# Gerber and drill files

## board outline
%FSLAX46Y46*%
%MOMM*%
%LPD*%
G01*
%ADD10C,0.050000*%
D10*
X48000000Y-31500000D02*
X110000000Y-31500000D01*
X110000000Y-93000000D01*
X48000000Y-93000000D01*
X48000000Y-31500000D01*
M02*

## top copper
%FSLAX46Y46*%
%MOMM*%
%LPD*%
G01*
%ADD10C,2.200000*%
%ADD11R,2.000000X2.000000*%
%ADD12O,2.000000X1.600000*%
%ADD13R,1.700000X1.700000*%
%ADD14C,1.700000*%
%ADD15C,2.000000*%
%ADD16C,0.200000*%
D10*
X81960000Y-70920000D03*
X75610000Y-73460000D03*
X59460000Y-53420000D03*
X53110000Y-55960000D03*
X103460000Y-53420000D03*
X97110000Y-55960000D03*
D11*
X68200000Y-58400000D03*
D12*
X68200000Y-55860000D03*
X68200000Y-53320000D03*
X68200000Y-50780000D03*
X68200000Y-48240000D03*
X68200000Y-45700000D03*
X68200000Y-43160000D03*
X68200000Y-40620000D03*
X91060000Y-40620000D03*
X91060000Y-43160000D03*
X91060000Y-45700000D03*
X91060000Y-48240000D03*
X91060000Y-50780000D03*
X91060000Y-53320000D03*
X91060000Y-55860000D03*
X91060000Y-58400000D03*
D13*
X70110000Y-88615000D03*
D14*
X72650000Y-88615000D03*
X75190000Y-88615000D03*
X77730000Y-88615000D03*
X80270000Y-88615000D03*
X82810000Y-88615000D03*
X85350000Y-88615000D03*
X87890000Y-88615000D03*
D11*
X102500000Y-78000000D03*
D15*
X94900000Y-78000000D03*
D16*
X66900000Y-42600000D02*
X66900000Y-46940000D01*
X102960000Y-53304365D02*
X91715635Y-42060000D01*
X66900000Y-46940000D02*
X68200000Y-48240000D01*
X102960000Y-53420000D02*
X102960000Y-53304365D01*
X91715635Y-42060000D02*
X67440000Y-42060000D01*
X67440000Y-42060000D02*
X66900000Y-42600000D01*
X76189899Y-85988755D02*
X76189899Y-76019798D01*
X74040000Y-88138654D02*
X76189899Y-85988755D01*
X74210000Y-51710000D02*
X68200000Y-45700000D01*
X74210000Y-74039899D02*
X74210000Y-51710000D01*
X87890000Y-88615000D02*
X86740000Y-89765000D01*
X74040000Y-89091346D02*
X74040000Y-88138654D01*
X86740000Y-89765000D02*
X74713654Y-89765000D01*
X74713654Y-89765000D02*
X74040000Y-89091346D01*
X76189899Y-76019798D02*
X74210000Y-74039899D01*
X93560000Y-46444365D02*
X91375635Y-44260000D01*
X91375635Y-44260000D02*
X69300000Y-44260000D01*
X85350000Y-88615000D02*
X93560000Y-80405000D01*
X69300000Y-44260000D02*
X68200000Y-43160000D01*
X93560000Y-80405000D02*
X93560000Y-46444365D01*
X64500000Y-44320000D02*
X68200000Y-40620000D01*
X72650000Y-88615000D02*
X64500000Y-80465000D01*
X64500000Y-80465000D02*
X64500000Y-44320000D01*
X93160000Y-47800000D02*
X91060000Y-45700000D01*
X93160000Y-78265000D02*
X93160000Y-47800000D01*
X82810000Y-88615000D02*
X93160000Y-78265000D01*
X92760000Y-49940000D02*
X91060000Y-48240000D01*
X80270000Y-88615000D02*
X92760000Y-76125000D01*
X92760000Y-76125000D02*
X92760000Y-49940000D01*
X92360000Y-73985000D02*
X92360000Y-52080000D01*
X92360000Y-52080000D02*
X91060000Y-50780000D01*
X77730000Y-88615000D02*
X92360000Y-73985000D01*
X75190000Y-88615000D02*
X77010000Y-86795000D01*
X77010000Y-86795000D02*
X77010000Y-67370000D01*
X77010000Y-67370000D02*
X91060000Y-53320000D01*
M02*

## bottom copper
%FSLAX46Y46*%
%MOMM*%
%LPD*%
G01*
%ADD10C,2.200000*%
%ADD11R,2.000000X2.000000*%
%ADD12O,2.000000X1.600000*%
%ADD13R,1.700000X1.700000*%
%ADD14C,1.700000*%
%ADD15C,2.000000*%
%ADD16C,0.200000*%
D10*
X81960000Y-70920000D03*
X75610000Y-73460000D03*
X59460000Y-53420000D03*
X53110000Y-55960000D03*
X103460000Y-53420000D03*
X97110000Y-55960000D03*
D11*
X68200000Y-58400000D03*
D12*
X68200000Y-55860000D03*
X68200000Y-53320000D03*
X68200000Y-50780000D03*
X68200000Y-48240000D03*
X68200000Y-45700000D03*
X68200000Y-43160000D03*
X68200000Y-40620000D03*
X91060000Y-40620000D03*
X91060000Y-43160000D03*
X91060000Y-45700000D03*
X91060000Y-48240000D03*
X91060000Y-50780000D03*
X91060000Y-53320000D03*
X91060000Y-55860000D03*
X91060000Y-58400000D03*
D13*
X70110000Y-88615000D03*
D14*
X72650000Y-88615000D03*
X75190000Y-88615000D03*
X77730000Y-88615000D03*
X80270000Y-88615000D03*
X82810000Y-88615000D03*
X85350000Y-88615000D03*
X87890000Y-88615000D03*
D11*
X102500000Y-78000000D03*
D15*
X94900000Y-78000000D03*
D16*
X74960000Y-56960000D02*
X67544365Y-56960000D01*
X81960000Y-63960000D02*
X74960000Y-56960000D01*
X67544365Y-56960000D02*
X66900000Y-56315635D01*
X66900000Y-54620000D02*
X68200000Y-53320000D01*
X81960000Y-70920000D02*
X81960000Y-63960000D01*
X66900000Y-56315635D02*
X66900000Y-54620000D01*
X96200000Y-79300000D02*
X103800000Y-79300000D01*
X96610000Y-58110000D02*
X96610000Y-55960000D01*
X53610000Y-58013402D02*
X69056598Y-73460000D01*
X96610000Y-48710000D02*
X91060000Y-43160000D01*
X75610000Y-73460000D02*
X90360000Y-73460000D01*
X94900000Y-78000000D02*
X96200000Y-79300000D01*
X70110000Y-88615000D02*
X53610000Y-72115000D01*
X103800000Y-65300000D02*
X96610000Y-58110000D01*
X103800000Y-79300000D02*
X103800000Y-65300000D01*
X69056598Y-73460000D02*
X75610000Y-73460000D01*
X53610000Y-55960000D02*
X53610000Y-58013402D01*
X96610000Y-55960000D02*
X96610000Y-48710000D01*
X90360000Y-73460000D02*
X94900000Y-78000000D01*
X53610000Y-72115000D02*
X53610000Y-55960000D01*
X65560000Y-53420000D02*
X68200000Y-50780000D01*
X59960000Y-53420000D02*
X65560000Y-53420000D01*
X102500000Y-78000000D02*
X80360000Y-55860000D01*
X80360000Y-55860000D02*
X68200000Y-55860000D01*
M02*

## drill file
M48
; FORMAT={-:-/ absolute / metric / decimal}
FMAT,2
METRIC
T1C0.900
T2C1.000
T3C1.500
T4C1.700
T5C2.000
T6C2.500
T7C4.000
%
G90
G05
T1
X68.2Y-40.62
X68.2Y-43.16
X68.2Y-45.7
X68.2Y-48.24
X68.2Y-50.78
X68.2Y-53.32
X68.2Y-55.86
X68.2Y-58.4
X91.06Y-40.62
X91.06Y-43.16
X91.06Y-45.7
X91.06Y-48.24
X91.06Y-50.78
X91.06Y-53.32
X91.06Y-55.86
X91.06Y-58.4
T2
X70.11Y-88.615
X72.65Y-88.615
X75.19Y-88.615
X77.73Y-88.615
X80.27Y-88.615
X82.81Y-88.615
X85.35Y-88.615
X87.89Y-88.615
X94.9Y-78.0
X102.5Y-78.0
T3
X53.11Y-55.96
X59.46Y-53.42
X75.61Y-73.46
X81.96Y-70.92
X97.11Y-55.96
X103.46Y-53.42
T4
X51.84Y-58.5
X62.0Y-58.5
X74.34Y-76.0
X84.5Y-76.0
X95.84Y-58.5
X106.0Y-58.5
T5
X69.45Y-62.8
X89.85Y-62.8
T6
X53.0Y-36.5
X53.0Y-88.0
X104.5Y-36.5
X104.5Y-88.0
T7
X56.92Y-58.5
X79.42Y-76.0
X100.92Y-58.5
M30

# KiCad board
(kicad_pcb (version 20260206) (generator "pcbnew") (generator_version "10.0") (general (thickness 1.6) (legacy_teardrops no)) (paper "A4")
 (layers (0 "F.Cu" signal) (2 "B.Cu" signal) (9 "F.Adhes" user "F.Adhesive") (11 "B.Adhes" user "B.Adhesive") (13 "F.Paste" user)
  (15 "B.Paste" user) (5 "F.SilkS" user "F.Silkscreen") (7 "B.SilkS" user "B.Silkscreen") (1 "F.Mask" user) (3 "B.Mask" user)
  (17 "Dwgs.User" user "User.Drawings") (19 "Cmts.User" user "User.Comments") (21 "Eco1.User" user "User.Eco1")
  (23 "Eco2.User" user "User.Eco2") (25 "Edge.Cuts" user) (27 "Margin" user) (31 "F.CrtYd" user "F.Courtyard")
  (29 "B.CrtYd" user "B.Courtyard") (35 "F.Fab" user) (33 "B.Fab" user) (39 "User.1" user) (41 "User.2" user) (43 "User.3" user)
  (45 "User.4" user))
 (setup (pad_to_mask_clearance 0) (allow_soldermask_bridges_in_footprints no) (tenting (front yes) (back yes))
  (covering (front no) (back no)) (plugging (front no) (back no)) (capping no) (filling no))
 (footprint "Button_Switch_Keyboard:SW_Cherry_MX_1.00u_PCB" (layer "F.Cu") (at 81.96 70.92)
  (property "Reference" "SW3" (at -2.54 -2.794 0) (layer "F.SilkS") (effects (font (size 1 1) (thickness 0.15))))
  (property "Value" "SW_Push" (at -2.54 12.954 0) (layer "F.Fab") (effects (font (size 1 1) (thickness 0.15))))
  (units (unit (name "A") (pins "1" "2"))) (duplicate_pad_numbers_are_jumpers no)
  (pad "" np_thru_hole circle (at -7.62 5.08) (size 1.7 1.7) (drill 1.7) (layers "*.Cu" "*.Mask"))
  (pad "" np_thru_hole circle (at -2.54 5.08) (size 4 4) (drill 4) (layers "*.Cu" "*.Mask"))
  (pad "" np_thru_hole circle (at 2.54 5.08) (size 1.7 1.7) (drill 1.7) (layers "*.Cu" "*.Mask"))
  (pad "1" thru_hole circle (at 0 0) (size 2.2 2.2) (drill 1.5) (layers "*.Cu" "*.Mask") (remove_unused_layers no) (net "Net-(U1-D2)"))
  (pad "2" thru_hole circle (at -6.35 2.54) (size 2.2 2.2) (drill 1.5) (layers "*.Cu" "*.Mask") (remove_unused_layers no) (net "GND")))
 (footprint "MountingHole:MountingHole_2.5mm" (layer "F.Cu") (at 104.5 36.5)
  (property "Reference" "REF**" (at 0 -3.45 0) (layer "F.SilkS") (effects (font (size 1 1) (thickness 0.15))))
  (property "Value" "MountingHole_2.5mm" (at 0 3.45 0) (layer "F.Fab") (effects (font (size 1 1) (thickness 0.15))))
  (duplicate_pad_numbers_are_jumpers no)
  (pad "" np_thru_hole circle (at 0 0) (size 2.5 2.5) (drill 2.5) (layers "*.Cu" "*.Mask")))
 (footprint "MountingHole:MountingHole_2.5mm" (layer "F.Cu") (at 53 36.5)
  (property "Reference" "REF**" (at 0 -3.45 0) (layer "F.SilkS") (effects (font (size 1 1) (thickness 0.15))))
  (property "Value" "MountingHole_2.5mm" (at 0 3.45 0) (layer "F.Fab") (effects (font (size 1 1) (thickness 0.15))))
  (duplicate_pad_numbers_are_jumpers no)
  (pad "" np_thru_hole circle (at 0 0) (size 2.5 2.5) (drill 2.5) (layers "*.Cu" "*.Mask")))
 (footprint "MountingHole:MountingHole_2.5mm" (layer "F.Cu") (at 104.5 88)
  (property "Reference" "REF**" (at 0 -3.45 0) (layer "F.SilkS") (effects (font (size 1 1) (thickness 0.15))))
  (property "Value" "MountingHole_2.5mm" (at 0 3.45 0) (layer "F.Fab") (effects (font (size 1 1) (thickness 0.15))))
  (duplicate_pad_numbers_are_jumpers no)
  (pad "" np_thru_hole circle (at 0 0) (size 2.5 2.5) (drill 2.5) (layers "*.Cu" "*.Mask")))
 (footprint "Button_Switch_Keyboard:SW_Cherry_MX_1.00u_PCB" (layer "F.Cu") (at 59.46 53.42)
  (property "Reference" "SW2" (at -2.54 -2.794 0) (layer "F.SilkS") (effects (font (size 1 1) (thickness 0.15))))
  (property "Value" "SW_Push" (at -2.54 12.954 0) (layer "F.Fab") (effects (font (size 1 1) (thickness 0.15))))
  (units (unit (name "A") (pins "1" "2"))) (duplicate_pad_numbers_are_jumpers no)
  (pad "" np_thru_hole circle (at -7.62 5.08) (size 1.7 1.7) (drill 1.7) (layers "*.Cu" "*.Mask"))
  (pad "" np_thru_hole circle (at -2.54 5.08) (size 4 4) (drill 4) (layers "*.Cu" "*.Mask"))
  (pad "" np_thru_hole circle (at 2.54 5.08) (size 1.7 1.7) (drill 1.7) (layers "*.Cu" "*.Mask"))
  (pad "1" thru_hole circle (at 0 0) (size 2.2 2.2) (drill 1.5) (layers "*.Cu" "*.Mask") (remove_unused_layers no) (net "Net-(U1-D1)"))
  (pad "2" thru_hole circle (at -6.35 2.54) (size 2.2 2.2) (drill 1.5) (layers "*.Cu" "*.Mask") (remove_unused_layers no) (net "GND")))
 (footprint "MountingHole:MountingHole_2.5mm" (layer "F.Cu") (at 53 88)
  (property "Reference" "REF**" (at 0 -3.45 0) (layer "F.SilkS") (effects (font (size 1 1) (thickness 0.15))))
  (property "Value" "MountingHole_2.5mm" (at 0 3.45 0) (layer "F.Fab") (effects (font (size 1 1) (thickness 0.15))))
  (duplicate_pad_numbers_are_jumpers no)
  (pad "" np_thru_hole circle (at 0 0) (size 2.5 2.5) (drill 2.5) (layers "*.Cu" "*.Mask")))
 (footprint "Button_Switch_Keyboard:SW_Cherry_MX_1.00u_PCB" (layer "F.Cu") (at 103.46 53.42)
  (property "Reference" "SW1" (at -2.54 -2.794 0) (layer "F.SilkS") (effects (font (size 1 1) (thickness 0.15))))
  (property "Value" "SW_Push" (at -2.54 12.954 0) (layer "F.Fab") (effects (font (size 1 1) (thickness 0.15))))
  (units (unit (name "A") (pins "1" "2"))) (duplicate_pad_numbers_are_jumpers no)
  (pad "" np_thru_hole circle (at -7.62 5.08) (size 1.7 1.7) (drill 1.7) (layers "*.Cu" "*.Mask"))
  (pad "" np_thru_hole circle (at -2.54 5.08) (size 4 4) (drill 4) (layers "*.Cu" "*.Mask"))
  (pad "" np_thru_hole circle (at 2.54 5.08) (size 1.7 1.7) (drill 1.7) (layers "*.Cu" "*.Mask"))
  (pad "1" thru_hole circle (at 0 0) (size 2.2 2.2) (drill 1.5) (layers "*.Cu" "*.Mask") (remove_unused_layers no) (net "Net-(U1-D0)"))
  (pad "2" thru_hole circle (at -6.35 2.54) (size 2.2 2.2) (drill 1.5) (layers "*.Cu" "*.Mask") (remove_unused_layers no) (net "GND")))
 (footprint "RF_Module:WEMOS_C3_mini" (layer "B.Cu") (at 68.2 58.4)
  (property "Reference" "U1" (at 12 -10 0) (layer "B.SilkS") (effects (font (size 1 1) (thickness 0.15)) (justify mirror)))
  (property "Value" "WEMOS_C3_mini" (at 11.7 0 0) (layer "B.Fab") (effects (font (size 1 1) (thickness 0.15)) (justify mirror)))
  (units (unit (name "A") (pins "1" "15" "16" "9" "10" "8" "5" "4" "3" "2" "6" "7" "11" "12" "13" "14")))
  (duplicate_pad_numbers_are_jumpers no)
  (pad "" np_thru_hole circle (at 1.25 4.4) (size 3 3) (drill 2) (layers "*.Mask"))
  (pad "" np_thru_hole circle (at 21.65 4.4) (size 3 3) (drill 2) (layers "*.Mask"))
  (pad "1" thru_hole rect (at 0 0) (size 2 2) (drill 0.9) (layers "*.Cu" "*.Mask") (remove_unused_layers no)
   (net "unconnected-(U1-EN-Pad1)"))
  (pad "2" thru_hole oval (at 0 -2.54) (size 2 1.6) (drill 0.9) (layers "*.Cu" "*.Mask") (remove_unused_layers no) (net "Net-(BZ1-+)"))
  (pad "3" thru_hole oval (at 0 -5.08) (size 2 1.6) (drill 0.9) (layers "*.Cu" "*.Mask") (remove_unused_layers no) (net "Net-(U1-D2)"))
  (pad "4" thru_hole oval (at 0 -7.62) (size 2 1.6) (drill 0.9) (layers "*.Cu" "*.Mask") (remove_unused_layers no) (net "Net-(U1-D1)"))
  (pad "5" thru_hole oval (at 0 -10.16) (size 2 1.6) (drill 0.9) (layers "*.Cu" "*.Mask") (remove_unused_layers no) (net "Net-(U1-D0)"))
  (pad "6" thru_hole oval (at 0 -12.7) (size 2 1.6) (drill 0.9) (layers "*.Cu" "*.Mask") (remove_unused_layers no) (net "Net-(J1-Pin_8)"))
  (pad "7" thru_hole oval (at 0 -15.24) (size 2 1.6) (drill 0.9) (layers "*.Cu" "*.Mask") (remove_unused_layers no) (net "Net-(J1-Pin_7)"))
  (pad "8" thru_hole oval (at 0 -17.78) (size 2 1.6) (drill 0.9) (layers "*.Cu" "*.Mask") (remove_unused_layers no) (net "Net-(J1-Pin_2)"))
  (pad "9" thru_hole oval (at 22.86 -17.78) (size 2 1.6) (drill 0.9) (layers "*.Cu" "*.Mask") (remove_unused_layers no)
   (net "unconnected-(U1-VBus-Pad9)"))
  (pad "10" thru_hole oval (at 22.86 -15.24) (size 2 1.6) (drill 0.9) (layers "*.Cu" "*.Mask") (remove_unused_layers no) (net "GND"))
  (pad "11" thru_hole oval (at 22.86 -12.7) (size 2 1.6) (drill 0.9) (layers "*.Cu" "*.Mask") (remove_unused_layers no)
   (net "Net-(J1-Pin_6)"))
  (pad "12" thru_hole oval (at 22.86 -10.16) (size 2 1.6) (drill 0.9) (layers "*.Cu" "*.Mask") (remove_unused_layers no)
   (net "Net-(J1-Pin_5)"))
  (pad "13" thru_hole oval (at 22.86 -7.62) (size 2 1.6) (drill 0.9) (layers "*.Cu" "*.Mask") (remove_unused_layers no)
   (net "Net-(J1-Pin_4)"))
  (pad "14" thru_hole oval (at 22.86 -5.08) (size 2 1.6) (drill 0.9) (layers "*.Cu" "*.Mask") (remove_unused_layers no)
   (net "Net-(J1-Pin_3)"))
  (pad "15" thru_hole oval (at 22.86 -2.54) (size 2 1.6) (drill 0.9) (layers "*.Cu" "*.Mask") (remove_unused_layers no)
   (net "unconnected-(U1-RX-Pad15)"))
  (pad "16" thru_hole oval (at 22.86 0) (size 2 1.6) (drill 0.9) (layers "*.Cu" "*.Mask") (remove_unused_layers no)
   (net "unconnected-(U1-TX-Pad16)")))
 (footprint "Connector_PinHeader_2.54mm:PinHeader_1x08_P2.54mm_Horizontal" (layer "B.Cu") (at 70.11 88.615 -90)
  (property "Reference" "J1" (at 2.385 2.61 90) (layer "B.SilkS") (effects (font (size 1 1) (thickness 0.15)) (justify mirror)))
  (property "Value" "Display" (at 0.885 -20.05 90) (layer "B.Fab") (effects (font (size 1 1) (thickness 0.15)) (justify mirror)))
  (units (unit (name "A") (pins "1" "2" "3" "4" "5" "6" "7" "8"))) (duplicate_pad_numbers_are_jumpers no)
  (pad "1" thru_hole rect (at 0 0 270) (size 1.7 1.7) (drill 1) (layers "*.Cu" "*.Mask") (remove_unused_layers no) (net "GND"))
  (pad "2" thru_hole circle (at 0 -2.54 270) (size 1.7 1.7) (drill 1) (layers "*.Cu" "*.Mask") (remove_unused_layers no)
   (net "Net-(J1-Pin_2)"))
  (pad "3" thru_hole circle (at 0 -5.08 270) (size 1.7 1.7) (drill 1) (layers "*.Cu" "*.Mask") (remove_unused_layers no)
   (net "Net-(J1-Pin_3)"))
  (pad "4" thru_hole circle (at 0 -7.62 270) (size 1.7 1.7) (drill 1) (layers "*.Cu" "*.Mask") (remove_unused_layers no)
   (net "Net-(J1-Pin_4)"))
  (pad "5" thru_hole circle (at 0 -10.16 270) (size 1.7 1.7) (drill 1) (layers "*.Cu" "*.Mask") (remove_unused_layers no)
   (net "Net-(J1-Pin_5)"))
  (pad "6" thru_hole circle (at 0 -12.7 270) (size 1.7 1.7) (drill 1) (layers "*.Cu" "*.Mask") (remove_unused_layers no)
   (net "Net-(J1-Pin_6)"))
  (pad "7" thru_hole circle (at 0 -15.24 270) (size 1.7 1.7) (drill 1) (layers "*.Cu" "*.Mask") (remove_unused_layers no)
   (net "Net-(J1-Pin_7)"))
  (pad "8" thru_hole circle (at 0 -17.78 270) (size 1.7 1.7) (drill 1) (layers "*.Cu" "*.Mask") (remove_unused_layers no)
   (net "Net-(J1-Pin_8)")))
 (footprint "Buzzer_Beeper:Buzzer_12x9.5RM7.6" (layer "B.Cu") (at 102.5 78 180)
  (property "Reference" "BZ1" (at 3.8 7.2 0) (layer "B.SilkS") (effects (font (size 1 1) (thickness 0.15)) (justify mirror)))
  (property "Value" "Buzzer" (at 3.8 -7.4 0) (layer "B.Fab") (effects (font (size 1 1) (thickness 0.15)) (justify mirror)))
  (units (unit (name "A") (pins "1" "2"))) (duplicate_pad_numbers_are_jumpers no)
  (pad "1" thru_hole rect (at 0 0 180) (size 2 2) (drill 1) (layers "*.Cu" "*.Mask") (remove_unused_layers no) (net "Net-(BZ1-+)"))
  (pad "2" thru_hole circle (at 7.6 0 180) (size 2 2) (drill 1) (layers "*.Cu" "*.Mask") (remove_unused_layers no) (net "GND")))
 (gr_rect (start 48 31.5) (end 110 93) (stroke (width 0.05) (type default)) (fill no) (layer "Edge.Cuts"))
 (segment (start 74.96 56.96) (end 67.544365 56.96) (width 0.2) (layer "B.Cu") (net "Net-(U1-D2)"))
 (segment (start 81.96 63.96) (end 74.96 56.96) (width 0.2) (layer "B.Cu") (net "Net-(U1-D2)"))
 (segment (start 67.544365 56.96) (end 66.9 56.315635) (width 0.2) (layer "B.Cu") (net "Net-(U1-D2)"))
 (segment (start 66.9 54.62) (end 68.2 53.32) (width 0.2) (layer "B.Cu") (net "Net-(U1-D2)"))
 (segment (start 81.96 70.92) (end 81.96 63.96) (width 0.2) (layer "B.Cu") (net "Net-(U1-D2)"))
 (segment (start 66.9 56.315635) (end 66.9 54.62) (width 0.2) (layer "B.Cu") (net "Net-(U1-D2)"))
 (segment (start 96.2 79.3) (end 103.8 79.3) (width 0.2) (layer "B.Cu") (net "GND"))
 (segment (start 96.61 58.11) (end 96.61 55.96) (width 0.2) (layer "B.Cu") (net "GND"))
 (segment (start 53.61 58.013402) (end 69.056598 73.46) (width 0.2) (layer "B.Cu") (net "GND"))
 (segment (start 96.61 48.71) (end 91.06 43.16) (width 0.2) (layer "B.Cu") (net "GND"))
 (segment (start 75.61 73.46) (end 90.36 73.46) (width 0.2) (layer "B.Cu") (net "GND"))
 (segment (start 94.9 78) (end 96.2 79.3) (width 0.2) (layer "B.Cu") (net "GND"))
 (segment (start 70.11 88.615) (end 53.61 72.115) (width 0.2) (layer "B.Cu") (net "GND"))
 (segment (start 103.8 65.3) (end 96.61 58.11) (width 0.2) (layer "B.Cu") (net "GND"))
 (segment (start 103.8 79.3) (end 103.8 65.3) (width 0.2) (layer "B.Cu") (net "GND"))
 (segment (start 69.056598 73.46) (end 75.61 73.46) (width 0.2) (layer "B.Cu") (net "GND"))
 (segment (start 53.61 55.96) (end 53.61 58.013402) (width 0.2) (layer "B.Cu") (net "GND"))
 (segment (start 96.61 55.96) (end 96.61 48.71) (width 0.2) (layer "B.Cu") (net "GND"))
 (segment (start 90.36 73.46) (end 94.9 78) (width 0.2) (layer "B.Cu") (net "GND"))
 (segment (start 53.61 72.115) (end 53.61 55.96) (width 0.2) (layer "B.Cu") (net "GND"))
 (segment (start 65.56 53.42) (end 68.2 50.78) (width 0.2) (layer "B.Cu") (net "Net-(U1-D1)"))
 (segment (start 59.96 53.42) (end 65.56 53.42) (width 0.2) (layer "B.Cu") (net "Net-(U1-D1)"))
 (segment (start 66.9 42.6) (end 66.9 46.94) (width 0.2) (layer "F.Cu") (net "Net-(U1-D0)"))
 (segment (start 102.96 53.304365) (end 91.715635 42.06) (width 0.2) (layer "F.Cu") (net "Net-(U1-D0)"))
 (segment (start 66.9 46.94) (end 68.2 48.24) (width 0.2) (layer "F.Cu") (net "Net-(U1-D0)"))
 (segment (start 102.96 53.42) (end 102.96 53.304365) (width 0.2) (layer "F.Cu") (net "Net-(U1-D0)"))
 (segment (start 91.715635 42.06) (end 67.44 42.06) (width 0.2) (layer "F.Cu") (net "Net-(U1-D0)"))
 (segment (start 67.44 42.06) (end 66.9 42.6) (width 0.2) (layer "F.Cu") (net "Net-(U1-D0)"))
 (segment (start 102.5 78) (end 80.36 55.86) (width 0.2) (layer "B.Cu") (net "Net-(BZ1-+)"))
 (segment (start 80.36 55.86) (end 68.2 55.86) (width 0.2) (layer "B.Cu") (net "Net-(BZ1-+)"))
 (segment (start 76.189899 85.988755) (end 76.189899 76.019798) (width 0.2) (layer "F.Cu") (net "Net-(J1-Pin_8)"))
 (segment (start 74.04 88.138654) (end 76.189899 85.988755) (width 0.2) (layer "F.Cu") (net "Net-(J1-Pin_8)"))
 (segment (start 74.21 51.71) (end 68.2 45.7) (width 0.2) (layer "F.Cu") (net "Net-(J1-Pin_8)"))
 (segment (start 74.21 74.039899) (end 74.21 51.71) (width 0.2) (layer "F.Cu") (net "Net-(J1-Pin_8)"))
 (segment (start 87.89 88.615) (end 86.74 89.765) (width 0.2) (layer "F.Cu") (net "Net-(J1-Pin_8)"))
 (segment (start 74.04 89.091346) (end 74.04 88.138654) (width 0.2) (layer "F.Cu") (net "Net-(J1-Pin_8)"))
 (segment (start 86.74 89.765) (end 74.713654 89.765) (width 0.2) (layer "F.Cu") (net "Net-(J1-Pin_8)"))
 (segment (start 74.713654 89.765) (end 74.04 89.091346) (width 0.2) (layer "F.Cu") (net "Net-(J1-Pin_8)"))
 (segment (start 76.189899 76.019798) (end 74.21 74.039899) (width 0.2) (layer "F.Cu") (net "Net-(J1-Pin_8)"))
 (segment (start 93.56 46.444365) (end 91.375635 44.26) (width 0.2) (layer "F.Cu") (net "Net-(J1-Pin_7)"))
 (segment (start 91.375635 44.26) (end 69.3 44.26) (width 0.2) (layer "F.Cu") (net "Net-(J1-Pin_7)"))
 (segment (start 85.35 88.615) (end 93.56 80.405) (width 0.2) (layer "F.Cu") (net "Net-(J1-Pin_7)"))
 (segment (start 69.3 44.26) (end 68.2 43.16) (width 0.2) (layer "F.Cu") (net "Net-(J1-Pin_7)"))
 (segment (start 93.56 80.405) (end 93.56 46.444365) (width 0.2) (layer "F.Cu") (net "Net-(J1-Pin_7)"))
 (segment (start 64.5 44.32) (end 68.2 40.62) (width 0.2) (layer "F.Cu") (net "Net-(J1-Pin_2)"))
 (segment (start 72.65 88.615) (end 64.5 80.465) (width 0.2) (layer "F.Cu") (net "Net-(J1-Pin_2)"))
 (segment (start 64.5 80.465) (end 64.5 44.32) (width 0.2) (layer "F.Cu") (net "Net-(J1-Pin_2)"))
 (segment (start 93.16 47.8) (end 91.06 45.7) (width 0.2) (layer "F.Cu") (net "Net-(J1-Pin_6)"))
 (segment (start 93.16 78.265) (end 93.16 47.8) (width 0.2) (layer "F.Cu") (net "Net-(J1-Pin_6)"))
 (segment (start 82.81 88.615) (end 93.16 78.265) (width 0.2) (layer "F.Cu") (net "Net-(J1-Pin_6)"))
 (segment (start 92.76 49.94) (end 91.06 48.24) (width 0.2) (layer "F.Cu") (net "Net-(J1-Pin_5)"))
 (segment (start 80.27 88.615) (end 92.76 76.125) (width 0.2) (layer "F.Cu") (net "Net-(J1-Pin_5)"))
 (segment (start 92.76 76.125) (end 92.76 49.94) (width 0.2) (layer "F.Cu") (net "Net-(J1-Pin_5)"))
 (segment (start 92.36 73.985) (end 92.36 52.08) (width 0.2) (layer "F.Cu") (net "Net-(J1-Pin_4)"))
 (segment (start 92.36 52.08) (end 91.06 50.78) (width 0.2) (layer "F.Cu") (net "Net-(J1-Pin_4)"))
 (segment (start 77.73 88.615) (end 92.36 73.985) (width 0.2) (layer "F.Cu") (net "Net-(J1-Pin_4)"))
 (segment (start 75.19 88.615) (end 77.01 86.795) (width 0.2) (layer "F.Cu") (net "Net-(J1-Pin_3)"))
 (segment (start 77.01 86.795) (end 77.01 67.37) (width 0.2) (layer "F.Cu") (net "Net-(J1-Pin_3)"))
 (segment (start 77.01 67.37) (end 91.06 53.32) (width 0.2) (layer "F.Cu") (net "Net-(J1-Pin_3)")))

